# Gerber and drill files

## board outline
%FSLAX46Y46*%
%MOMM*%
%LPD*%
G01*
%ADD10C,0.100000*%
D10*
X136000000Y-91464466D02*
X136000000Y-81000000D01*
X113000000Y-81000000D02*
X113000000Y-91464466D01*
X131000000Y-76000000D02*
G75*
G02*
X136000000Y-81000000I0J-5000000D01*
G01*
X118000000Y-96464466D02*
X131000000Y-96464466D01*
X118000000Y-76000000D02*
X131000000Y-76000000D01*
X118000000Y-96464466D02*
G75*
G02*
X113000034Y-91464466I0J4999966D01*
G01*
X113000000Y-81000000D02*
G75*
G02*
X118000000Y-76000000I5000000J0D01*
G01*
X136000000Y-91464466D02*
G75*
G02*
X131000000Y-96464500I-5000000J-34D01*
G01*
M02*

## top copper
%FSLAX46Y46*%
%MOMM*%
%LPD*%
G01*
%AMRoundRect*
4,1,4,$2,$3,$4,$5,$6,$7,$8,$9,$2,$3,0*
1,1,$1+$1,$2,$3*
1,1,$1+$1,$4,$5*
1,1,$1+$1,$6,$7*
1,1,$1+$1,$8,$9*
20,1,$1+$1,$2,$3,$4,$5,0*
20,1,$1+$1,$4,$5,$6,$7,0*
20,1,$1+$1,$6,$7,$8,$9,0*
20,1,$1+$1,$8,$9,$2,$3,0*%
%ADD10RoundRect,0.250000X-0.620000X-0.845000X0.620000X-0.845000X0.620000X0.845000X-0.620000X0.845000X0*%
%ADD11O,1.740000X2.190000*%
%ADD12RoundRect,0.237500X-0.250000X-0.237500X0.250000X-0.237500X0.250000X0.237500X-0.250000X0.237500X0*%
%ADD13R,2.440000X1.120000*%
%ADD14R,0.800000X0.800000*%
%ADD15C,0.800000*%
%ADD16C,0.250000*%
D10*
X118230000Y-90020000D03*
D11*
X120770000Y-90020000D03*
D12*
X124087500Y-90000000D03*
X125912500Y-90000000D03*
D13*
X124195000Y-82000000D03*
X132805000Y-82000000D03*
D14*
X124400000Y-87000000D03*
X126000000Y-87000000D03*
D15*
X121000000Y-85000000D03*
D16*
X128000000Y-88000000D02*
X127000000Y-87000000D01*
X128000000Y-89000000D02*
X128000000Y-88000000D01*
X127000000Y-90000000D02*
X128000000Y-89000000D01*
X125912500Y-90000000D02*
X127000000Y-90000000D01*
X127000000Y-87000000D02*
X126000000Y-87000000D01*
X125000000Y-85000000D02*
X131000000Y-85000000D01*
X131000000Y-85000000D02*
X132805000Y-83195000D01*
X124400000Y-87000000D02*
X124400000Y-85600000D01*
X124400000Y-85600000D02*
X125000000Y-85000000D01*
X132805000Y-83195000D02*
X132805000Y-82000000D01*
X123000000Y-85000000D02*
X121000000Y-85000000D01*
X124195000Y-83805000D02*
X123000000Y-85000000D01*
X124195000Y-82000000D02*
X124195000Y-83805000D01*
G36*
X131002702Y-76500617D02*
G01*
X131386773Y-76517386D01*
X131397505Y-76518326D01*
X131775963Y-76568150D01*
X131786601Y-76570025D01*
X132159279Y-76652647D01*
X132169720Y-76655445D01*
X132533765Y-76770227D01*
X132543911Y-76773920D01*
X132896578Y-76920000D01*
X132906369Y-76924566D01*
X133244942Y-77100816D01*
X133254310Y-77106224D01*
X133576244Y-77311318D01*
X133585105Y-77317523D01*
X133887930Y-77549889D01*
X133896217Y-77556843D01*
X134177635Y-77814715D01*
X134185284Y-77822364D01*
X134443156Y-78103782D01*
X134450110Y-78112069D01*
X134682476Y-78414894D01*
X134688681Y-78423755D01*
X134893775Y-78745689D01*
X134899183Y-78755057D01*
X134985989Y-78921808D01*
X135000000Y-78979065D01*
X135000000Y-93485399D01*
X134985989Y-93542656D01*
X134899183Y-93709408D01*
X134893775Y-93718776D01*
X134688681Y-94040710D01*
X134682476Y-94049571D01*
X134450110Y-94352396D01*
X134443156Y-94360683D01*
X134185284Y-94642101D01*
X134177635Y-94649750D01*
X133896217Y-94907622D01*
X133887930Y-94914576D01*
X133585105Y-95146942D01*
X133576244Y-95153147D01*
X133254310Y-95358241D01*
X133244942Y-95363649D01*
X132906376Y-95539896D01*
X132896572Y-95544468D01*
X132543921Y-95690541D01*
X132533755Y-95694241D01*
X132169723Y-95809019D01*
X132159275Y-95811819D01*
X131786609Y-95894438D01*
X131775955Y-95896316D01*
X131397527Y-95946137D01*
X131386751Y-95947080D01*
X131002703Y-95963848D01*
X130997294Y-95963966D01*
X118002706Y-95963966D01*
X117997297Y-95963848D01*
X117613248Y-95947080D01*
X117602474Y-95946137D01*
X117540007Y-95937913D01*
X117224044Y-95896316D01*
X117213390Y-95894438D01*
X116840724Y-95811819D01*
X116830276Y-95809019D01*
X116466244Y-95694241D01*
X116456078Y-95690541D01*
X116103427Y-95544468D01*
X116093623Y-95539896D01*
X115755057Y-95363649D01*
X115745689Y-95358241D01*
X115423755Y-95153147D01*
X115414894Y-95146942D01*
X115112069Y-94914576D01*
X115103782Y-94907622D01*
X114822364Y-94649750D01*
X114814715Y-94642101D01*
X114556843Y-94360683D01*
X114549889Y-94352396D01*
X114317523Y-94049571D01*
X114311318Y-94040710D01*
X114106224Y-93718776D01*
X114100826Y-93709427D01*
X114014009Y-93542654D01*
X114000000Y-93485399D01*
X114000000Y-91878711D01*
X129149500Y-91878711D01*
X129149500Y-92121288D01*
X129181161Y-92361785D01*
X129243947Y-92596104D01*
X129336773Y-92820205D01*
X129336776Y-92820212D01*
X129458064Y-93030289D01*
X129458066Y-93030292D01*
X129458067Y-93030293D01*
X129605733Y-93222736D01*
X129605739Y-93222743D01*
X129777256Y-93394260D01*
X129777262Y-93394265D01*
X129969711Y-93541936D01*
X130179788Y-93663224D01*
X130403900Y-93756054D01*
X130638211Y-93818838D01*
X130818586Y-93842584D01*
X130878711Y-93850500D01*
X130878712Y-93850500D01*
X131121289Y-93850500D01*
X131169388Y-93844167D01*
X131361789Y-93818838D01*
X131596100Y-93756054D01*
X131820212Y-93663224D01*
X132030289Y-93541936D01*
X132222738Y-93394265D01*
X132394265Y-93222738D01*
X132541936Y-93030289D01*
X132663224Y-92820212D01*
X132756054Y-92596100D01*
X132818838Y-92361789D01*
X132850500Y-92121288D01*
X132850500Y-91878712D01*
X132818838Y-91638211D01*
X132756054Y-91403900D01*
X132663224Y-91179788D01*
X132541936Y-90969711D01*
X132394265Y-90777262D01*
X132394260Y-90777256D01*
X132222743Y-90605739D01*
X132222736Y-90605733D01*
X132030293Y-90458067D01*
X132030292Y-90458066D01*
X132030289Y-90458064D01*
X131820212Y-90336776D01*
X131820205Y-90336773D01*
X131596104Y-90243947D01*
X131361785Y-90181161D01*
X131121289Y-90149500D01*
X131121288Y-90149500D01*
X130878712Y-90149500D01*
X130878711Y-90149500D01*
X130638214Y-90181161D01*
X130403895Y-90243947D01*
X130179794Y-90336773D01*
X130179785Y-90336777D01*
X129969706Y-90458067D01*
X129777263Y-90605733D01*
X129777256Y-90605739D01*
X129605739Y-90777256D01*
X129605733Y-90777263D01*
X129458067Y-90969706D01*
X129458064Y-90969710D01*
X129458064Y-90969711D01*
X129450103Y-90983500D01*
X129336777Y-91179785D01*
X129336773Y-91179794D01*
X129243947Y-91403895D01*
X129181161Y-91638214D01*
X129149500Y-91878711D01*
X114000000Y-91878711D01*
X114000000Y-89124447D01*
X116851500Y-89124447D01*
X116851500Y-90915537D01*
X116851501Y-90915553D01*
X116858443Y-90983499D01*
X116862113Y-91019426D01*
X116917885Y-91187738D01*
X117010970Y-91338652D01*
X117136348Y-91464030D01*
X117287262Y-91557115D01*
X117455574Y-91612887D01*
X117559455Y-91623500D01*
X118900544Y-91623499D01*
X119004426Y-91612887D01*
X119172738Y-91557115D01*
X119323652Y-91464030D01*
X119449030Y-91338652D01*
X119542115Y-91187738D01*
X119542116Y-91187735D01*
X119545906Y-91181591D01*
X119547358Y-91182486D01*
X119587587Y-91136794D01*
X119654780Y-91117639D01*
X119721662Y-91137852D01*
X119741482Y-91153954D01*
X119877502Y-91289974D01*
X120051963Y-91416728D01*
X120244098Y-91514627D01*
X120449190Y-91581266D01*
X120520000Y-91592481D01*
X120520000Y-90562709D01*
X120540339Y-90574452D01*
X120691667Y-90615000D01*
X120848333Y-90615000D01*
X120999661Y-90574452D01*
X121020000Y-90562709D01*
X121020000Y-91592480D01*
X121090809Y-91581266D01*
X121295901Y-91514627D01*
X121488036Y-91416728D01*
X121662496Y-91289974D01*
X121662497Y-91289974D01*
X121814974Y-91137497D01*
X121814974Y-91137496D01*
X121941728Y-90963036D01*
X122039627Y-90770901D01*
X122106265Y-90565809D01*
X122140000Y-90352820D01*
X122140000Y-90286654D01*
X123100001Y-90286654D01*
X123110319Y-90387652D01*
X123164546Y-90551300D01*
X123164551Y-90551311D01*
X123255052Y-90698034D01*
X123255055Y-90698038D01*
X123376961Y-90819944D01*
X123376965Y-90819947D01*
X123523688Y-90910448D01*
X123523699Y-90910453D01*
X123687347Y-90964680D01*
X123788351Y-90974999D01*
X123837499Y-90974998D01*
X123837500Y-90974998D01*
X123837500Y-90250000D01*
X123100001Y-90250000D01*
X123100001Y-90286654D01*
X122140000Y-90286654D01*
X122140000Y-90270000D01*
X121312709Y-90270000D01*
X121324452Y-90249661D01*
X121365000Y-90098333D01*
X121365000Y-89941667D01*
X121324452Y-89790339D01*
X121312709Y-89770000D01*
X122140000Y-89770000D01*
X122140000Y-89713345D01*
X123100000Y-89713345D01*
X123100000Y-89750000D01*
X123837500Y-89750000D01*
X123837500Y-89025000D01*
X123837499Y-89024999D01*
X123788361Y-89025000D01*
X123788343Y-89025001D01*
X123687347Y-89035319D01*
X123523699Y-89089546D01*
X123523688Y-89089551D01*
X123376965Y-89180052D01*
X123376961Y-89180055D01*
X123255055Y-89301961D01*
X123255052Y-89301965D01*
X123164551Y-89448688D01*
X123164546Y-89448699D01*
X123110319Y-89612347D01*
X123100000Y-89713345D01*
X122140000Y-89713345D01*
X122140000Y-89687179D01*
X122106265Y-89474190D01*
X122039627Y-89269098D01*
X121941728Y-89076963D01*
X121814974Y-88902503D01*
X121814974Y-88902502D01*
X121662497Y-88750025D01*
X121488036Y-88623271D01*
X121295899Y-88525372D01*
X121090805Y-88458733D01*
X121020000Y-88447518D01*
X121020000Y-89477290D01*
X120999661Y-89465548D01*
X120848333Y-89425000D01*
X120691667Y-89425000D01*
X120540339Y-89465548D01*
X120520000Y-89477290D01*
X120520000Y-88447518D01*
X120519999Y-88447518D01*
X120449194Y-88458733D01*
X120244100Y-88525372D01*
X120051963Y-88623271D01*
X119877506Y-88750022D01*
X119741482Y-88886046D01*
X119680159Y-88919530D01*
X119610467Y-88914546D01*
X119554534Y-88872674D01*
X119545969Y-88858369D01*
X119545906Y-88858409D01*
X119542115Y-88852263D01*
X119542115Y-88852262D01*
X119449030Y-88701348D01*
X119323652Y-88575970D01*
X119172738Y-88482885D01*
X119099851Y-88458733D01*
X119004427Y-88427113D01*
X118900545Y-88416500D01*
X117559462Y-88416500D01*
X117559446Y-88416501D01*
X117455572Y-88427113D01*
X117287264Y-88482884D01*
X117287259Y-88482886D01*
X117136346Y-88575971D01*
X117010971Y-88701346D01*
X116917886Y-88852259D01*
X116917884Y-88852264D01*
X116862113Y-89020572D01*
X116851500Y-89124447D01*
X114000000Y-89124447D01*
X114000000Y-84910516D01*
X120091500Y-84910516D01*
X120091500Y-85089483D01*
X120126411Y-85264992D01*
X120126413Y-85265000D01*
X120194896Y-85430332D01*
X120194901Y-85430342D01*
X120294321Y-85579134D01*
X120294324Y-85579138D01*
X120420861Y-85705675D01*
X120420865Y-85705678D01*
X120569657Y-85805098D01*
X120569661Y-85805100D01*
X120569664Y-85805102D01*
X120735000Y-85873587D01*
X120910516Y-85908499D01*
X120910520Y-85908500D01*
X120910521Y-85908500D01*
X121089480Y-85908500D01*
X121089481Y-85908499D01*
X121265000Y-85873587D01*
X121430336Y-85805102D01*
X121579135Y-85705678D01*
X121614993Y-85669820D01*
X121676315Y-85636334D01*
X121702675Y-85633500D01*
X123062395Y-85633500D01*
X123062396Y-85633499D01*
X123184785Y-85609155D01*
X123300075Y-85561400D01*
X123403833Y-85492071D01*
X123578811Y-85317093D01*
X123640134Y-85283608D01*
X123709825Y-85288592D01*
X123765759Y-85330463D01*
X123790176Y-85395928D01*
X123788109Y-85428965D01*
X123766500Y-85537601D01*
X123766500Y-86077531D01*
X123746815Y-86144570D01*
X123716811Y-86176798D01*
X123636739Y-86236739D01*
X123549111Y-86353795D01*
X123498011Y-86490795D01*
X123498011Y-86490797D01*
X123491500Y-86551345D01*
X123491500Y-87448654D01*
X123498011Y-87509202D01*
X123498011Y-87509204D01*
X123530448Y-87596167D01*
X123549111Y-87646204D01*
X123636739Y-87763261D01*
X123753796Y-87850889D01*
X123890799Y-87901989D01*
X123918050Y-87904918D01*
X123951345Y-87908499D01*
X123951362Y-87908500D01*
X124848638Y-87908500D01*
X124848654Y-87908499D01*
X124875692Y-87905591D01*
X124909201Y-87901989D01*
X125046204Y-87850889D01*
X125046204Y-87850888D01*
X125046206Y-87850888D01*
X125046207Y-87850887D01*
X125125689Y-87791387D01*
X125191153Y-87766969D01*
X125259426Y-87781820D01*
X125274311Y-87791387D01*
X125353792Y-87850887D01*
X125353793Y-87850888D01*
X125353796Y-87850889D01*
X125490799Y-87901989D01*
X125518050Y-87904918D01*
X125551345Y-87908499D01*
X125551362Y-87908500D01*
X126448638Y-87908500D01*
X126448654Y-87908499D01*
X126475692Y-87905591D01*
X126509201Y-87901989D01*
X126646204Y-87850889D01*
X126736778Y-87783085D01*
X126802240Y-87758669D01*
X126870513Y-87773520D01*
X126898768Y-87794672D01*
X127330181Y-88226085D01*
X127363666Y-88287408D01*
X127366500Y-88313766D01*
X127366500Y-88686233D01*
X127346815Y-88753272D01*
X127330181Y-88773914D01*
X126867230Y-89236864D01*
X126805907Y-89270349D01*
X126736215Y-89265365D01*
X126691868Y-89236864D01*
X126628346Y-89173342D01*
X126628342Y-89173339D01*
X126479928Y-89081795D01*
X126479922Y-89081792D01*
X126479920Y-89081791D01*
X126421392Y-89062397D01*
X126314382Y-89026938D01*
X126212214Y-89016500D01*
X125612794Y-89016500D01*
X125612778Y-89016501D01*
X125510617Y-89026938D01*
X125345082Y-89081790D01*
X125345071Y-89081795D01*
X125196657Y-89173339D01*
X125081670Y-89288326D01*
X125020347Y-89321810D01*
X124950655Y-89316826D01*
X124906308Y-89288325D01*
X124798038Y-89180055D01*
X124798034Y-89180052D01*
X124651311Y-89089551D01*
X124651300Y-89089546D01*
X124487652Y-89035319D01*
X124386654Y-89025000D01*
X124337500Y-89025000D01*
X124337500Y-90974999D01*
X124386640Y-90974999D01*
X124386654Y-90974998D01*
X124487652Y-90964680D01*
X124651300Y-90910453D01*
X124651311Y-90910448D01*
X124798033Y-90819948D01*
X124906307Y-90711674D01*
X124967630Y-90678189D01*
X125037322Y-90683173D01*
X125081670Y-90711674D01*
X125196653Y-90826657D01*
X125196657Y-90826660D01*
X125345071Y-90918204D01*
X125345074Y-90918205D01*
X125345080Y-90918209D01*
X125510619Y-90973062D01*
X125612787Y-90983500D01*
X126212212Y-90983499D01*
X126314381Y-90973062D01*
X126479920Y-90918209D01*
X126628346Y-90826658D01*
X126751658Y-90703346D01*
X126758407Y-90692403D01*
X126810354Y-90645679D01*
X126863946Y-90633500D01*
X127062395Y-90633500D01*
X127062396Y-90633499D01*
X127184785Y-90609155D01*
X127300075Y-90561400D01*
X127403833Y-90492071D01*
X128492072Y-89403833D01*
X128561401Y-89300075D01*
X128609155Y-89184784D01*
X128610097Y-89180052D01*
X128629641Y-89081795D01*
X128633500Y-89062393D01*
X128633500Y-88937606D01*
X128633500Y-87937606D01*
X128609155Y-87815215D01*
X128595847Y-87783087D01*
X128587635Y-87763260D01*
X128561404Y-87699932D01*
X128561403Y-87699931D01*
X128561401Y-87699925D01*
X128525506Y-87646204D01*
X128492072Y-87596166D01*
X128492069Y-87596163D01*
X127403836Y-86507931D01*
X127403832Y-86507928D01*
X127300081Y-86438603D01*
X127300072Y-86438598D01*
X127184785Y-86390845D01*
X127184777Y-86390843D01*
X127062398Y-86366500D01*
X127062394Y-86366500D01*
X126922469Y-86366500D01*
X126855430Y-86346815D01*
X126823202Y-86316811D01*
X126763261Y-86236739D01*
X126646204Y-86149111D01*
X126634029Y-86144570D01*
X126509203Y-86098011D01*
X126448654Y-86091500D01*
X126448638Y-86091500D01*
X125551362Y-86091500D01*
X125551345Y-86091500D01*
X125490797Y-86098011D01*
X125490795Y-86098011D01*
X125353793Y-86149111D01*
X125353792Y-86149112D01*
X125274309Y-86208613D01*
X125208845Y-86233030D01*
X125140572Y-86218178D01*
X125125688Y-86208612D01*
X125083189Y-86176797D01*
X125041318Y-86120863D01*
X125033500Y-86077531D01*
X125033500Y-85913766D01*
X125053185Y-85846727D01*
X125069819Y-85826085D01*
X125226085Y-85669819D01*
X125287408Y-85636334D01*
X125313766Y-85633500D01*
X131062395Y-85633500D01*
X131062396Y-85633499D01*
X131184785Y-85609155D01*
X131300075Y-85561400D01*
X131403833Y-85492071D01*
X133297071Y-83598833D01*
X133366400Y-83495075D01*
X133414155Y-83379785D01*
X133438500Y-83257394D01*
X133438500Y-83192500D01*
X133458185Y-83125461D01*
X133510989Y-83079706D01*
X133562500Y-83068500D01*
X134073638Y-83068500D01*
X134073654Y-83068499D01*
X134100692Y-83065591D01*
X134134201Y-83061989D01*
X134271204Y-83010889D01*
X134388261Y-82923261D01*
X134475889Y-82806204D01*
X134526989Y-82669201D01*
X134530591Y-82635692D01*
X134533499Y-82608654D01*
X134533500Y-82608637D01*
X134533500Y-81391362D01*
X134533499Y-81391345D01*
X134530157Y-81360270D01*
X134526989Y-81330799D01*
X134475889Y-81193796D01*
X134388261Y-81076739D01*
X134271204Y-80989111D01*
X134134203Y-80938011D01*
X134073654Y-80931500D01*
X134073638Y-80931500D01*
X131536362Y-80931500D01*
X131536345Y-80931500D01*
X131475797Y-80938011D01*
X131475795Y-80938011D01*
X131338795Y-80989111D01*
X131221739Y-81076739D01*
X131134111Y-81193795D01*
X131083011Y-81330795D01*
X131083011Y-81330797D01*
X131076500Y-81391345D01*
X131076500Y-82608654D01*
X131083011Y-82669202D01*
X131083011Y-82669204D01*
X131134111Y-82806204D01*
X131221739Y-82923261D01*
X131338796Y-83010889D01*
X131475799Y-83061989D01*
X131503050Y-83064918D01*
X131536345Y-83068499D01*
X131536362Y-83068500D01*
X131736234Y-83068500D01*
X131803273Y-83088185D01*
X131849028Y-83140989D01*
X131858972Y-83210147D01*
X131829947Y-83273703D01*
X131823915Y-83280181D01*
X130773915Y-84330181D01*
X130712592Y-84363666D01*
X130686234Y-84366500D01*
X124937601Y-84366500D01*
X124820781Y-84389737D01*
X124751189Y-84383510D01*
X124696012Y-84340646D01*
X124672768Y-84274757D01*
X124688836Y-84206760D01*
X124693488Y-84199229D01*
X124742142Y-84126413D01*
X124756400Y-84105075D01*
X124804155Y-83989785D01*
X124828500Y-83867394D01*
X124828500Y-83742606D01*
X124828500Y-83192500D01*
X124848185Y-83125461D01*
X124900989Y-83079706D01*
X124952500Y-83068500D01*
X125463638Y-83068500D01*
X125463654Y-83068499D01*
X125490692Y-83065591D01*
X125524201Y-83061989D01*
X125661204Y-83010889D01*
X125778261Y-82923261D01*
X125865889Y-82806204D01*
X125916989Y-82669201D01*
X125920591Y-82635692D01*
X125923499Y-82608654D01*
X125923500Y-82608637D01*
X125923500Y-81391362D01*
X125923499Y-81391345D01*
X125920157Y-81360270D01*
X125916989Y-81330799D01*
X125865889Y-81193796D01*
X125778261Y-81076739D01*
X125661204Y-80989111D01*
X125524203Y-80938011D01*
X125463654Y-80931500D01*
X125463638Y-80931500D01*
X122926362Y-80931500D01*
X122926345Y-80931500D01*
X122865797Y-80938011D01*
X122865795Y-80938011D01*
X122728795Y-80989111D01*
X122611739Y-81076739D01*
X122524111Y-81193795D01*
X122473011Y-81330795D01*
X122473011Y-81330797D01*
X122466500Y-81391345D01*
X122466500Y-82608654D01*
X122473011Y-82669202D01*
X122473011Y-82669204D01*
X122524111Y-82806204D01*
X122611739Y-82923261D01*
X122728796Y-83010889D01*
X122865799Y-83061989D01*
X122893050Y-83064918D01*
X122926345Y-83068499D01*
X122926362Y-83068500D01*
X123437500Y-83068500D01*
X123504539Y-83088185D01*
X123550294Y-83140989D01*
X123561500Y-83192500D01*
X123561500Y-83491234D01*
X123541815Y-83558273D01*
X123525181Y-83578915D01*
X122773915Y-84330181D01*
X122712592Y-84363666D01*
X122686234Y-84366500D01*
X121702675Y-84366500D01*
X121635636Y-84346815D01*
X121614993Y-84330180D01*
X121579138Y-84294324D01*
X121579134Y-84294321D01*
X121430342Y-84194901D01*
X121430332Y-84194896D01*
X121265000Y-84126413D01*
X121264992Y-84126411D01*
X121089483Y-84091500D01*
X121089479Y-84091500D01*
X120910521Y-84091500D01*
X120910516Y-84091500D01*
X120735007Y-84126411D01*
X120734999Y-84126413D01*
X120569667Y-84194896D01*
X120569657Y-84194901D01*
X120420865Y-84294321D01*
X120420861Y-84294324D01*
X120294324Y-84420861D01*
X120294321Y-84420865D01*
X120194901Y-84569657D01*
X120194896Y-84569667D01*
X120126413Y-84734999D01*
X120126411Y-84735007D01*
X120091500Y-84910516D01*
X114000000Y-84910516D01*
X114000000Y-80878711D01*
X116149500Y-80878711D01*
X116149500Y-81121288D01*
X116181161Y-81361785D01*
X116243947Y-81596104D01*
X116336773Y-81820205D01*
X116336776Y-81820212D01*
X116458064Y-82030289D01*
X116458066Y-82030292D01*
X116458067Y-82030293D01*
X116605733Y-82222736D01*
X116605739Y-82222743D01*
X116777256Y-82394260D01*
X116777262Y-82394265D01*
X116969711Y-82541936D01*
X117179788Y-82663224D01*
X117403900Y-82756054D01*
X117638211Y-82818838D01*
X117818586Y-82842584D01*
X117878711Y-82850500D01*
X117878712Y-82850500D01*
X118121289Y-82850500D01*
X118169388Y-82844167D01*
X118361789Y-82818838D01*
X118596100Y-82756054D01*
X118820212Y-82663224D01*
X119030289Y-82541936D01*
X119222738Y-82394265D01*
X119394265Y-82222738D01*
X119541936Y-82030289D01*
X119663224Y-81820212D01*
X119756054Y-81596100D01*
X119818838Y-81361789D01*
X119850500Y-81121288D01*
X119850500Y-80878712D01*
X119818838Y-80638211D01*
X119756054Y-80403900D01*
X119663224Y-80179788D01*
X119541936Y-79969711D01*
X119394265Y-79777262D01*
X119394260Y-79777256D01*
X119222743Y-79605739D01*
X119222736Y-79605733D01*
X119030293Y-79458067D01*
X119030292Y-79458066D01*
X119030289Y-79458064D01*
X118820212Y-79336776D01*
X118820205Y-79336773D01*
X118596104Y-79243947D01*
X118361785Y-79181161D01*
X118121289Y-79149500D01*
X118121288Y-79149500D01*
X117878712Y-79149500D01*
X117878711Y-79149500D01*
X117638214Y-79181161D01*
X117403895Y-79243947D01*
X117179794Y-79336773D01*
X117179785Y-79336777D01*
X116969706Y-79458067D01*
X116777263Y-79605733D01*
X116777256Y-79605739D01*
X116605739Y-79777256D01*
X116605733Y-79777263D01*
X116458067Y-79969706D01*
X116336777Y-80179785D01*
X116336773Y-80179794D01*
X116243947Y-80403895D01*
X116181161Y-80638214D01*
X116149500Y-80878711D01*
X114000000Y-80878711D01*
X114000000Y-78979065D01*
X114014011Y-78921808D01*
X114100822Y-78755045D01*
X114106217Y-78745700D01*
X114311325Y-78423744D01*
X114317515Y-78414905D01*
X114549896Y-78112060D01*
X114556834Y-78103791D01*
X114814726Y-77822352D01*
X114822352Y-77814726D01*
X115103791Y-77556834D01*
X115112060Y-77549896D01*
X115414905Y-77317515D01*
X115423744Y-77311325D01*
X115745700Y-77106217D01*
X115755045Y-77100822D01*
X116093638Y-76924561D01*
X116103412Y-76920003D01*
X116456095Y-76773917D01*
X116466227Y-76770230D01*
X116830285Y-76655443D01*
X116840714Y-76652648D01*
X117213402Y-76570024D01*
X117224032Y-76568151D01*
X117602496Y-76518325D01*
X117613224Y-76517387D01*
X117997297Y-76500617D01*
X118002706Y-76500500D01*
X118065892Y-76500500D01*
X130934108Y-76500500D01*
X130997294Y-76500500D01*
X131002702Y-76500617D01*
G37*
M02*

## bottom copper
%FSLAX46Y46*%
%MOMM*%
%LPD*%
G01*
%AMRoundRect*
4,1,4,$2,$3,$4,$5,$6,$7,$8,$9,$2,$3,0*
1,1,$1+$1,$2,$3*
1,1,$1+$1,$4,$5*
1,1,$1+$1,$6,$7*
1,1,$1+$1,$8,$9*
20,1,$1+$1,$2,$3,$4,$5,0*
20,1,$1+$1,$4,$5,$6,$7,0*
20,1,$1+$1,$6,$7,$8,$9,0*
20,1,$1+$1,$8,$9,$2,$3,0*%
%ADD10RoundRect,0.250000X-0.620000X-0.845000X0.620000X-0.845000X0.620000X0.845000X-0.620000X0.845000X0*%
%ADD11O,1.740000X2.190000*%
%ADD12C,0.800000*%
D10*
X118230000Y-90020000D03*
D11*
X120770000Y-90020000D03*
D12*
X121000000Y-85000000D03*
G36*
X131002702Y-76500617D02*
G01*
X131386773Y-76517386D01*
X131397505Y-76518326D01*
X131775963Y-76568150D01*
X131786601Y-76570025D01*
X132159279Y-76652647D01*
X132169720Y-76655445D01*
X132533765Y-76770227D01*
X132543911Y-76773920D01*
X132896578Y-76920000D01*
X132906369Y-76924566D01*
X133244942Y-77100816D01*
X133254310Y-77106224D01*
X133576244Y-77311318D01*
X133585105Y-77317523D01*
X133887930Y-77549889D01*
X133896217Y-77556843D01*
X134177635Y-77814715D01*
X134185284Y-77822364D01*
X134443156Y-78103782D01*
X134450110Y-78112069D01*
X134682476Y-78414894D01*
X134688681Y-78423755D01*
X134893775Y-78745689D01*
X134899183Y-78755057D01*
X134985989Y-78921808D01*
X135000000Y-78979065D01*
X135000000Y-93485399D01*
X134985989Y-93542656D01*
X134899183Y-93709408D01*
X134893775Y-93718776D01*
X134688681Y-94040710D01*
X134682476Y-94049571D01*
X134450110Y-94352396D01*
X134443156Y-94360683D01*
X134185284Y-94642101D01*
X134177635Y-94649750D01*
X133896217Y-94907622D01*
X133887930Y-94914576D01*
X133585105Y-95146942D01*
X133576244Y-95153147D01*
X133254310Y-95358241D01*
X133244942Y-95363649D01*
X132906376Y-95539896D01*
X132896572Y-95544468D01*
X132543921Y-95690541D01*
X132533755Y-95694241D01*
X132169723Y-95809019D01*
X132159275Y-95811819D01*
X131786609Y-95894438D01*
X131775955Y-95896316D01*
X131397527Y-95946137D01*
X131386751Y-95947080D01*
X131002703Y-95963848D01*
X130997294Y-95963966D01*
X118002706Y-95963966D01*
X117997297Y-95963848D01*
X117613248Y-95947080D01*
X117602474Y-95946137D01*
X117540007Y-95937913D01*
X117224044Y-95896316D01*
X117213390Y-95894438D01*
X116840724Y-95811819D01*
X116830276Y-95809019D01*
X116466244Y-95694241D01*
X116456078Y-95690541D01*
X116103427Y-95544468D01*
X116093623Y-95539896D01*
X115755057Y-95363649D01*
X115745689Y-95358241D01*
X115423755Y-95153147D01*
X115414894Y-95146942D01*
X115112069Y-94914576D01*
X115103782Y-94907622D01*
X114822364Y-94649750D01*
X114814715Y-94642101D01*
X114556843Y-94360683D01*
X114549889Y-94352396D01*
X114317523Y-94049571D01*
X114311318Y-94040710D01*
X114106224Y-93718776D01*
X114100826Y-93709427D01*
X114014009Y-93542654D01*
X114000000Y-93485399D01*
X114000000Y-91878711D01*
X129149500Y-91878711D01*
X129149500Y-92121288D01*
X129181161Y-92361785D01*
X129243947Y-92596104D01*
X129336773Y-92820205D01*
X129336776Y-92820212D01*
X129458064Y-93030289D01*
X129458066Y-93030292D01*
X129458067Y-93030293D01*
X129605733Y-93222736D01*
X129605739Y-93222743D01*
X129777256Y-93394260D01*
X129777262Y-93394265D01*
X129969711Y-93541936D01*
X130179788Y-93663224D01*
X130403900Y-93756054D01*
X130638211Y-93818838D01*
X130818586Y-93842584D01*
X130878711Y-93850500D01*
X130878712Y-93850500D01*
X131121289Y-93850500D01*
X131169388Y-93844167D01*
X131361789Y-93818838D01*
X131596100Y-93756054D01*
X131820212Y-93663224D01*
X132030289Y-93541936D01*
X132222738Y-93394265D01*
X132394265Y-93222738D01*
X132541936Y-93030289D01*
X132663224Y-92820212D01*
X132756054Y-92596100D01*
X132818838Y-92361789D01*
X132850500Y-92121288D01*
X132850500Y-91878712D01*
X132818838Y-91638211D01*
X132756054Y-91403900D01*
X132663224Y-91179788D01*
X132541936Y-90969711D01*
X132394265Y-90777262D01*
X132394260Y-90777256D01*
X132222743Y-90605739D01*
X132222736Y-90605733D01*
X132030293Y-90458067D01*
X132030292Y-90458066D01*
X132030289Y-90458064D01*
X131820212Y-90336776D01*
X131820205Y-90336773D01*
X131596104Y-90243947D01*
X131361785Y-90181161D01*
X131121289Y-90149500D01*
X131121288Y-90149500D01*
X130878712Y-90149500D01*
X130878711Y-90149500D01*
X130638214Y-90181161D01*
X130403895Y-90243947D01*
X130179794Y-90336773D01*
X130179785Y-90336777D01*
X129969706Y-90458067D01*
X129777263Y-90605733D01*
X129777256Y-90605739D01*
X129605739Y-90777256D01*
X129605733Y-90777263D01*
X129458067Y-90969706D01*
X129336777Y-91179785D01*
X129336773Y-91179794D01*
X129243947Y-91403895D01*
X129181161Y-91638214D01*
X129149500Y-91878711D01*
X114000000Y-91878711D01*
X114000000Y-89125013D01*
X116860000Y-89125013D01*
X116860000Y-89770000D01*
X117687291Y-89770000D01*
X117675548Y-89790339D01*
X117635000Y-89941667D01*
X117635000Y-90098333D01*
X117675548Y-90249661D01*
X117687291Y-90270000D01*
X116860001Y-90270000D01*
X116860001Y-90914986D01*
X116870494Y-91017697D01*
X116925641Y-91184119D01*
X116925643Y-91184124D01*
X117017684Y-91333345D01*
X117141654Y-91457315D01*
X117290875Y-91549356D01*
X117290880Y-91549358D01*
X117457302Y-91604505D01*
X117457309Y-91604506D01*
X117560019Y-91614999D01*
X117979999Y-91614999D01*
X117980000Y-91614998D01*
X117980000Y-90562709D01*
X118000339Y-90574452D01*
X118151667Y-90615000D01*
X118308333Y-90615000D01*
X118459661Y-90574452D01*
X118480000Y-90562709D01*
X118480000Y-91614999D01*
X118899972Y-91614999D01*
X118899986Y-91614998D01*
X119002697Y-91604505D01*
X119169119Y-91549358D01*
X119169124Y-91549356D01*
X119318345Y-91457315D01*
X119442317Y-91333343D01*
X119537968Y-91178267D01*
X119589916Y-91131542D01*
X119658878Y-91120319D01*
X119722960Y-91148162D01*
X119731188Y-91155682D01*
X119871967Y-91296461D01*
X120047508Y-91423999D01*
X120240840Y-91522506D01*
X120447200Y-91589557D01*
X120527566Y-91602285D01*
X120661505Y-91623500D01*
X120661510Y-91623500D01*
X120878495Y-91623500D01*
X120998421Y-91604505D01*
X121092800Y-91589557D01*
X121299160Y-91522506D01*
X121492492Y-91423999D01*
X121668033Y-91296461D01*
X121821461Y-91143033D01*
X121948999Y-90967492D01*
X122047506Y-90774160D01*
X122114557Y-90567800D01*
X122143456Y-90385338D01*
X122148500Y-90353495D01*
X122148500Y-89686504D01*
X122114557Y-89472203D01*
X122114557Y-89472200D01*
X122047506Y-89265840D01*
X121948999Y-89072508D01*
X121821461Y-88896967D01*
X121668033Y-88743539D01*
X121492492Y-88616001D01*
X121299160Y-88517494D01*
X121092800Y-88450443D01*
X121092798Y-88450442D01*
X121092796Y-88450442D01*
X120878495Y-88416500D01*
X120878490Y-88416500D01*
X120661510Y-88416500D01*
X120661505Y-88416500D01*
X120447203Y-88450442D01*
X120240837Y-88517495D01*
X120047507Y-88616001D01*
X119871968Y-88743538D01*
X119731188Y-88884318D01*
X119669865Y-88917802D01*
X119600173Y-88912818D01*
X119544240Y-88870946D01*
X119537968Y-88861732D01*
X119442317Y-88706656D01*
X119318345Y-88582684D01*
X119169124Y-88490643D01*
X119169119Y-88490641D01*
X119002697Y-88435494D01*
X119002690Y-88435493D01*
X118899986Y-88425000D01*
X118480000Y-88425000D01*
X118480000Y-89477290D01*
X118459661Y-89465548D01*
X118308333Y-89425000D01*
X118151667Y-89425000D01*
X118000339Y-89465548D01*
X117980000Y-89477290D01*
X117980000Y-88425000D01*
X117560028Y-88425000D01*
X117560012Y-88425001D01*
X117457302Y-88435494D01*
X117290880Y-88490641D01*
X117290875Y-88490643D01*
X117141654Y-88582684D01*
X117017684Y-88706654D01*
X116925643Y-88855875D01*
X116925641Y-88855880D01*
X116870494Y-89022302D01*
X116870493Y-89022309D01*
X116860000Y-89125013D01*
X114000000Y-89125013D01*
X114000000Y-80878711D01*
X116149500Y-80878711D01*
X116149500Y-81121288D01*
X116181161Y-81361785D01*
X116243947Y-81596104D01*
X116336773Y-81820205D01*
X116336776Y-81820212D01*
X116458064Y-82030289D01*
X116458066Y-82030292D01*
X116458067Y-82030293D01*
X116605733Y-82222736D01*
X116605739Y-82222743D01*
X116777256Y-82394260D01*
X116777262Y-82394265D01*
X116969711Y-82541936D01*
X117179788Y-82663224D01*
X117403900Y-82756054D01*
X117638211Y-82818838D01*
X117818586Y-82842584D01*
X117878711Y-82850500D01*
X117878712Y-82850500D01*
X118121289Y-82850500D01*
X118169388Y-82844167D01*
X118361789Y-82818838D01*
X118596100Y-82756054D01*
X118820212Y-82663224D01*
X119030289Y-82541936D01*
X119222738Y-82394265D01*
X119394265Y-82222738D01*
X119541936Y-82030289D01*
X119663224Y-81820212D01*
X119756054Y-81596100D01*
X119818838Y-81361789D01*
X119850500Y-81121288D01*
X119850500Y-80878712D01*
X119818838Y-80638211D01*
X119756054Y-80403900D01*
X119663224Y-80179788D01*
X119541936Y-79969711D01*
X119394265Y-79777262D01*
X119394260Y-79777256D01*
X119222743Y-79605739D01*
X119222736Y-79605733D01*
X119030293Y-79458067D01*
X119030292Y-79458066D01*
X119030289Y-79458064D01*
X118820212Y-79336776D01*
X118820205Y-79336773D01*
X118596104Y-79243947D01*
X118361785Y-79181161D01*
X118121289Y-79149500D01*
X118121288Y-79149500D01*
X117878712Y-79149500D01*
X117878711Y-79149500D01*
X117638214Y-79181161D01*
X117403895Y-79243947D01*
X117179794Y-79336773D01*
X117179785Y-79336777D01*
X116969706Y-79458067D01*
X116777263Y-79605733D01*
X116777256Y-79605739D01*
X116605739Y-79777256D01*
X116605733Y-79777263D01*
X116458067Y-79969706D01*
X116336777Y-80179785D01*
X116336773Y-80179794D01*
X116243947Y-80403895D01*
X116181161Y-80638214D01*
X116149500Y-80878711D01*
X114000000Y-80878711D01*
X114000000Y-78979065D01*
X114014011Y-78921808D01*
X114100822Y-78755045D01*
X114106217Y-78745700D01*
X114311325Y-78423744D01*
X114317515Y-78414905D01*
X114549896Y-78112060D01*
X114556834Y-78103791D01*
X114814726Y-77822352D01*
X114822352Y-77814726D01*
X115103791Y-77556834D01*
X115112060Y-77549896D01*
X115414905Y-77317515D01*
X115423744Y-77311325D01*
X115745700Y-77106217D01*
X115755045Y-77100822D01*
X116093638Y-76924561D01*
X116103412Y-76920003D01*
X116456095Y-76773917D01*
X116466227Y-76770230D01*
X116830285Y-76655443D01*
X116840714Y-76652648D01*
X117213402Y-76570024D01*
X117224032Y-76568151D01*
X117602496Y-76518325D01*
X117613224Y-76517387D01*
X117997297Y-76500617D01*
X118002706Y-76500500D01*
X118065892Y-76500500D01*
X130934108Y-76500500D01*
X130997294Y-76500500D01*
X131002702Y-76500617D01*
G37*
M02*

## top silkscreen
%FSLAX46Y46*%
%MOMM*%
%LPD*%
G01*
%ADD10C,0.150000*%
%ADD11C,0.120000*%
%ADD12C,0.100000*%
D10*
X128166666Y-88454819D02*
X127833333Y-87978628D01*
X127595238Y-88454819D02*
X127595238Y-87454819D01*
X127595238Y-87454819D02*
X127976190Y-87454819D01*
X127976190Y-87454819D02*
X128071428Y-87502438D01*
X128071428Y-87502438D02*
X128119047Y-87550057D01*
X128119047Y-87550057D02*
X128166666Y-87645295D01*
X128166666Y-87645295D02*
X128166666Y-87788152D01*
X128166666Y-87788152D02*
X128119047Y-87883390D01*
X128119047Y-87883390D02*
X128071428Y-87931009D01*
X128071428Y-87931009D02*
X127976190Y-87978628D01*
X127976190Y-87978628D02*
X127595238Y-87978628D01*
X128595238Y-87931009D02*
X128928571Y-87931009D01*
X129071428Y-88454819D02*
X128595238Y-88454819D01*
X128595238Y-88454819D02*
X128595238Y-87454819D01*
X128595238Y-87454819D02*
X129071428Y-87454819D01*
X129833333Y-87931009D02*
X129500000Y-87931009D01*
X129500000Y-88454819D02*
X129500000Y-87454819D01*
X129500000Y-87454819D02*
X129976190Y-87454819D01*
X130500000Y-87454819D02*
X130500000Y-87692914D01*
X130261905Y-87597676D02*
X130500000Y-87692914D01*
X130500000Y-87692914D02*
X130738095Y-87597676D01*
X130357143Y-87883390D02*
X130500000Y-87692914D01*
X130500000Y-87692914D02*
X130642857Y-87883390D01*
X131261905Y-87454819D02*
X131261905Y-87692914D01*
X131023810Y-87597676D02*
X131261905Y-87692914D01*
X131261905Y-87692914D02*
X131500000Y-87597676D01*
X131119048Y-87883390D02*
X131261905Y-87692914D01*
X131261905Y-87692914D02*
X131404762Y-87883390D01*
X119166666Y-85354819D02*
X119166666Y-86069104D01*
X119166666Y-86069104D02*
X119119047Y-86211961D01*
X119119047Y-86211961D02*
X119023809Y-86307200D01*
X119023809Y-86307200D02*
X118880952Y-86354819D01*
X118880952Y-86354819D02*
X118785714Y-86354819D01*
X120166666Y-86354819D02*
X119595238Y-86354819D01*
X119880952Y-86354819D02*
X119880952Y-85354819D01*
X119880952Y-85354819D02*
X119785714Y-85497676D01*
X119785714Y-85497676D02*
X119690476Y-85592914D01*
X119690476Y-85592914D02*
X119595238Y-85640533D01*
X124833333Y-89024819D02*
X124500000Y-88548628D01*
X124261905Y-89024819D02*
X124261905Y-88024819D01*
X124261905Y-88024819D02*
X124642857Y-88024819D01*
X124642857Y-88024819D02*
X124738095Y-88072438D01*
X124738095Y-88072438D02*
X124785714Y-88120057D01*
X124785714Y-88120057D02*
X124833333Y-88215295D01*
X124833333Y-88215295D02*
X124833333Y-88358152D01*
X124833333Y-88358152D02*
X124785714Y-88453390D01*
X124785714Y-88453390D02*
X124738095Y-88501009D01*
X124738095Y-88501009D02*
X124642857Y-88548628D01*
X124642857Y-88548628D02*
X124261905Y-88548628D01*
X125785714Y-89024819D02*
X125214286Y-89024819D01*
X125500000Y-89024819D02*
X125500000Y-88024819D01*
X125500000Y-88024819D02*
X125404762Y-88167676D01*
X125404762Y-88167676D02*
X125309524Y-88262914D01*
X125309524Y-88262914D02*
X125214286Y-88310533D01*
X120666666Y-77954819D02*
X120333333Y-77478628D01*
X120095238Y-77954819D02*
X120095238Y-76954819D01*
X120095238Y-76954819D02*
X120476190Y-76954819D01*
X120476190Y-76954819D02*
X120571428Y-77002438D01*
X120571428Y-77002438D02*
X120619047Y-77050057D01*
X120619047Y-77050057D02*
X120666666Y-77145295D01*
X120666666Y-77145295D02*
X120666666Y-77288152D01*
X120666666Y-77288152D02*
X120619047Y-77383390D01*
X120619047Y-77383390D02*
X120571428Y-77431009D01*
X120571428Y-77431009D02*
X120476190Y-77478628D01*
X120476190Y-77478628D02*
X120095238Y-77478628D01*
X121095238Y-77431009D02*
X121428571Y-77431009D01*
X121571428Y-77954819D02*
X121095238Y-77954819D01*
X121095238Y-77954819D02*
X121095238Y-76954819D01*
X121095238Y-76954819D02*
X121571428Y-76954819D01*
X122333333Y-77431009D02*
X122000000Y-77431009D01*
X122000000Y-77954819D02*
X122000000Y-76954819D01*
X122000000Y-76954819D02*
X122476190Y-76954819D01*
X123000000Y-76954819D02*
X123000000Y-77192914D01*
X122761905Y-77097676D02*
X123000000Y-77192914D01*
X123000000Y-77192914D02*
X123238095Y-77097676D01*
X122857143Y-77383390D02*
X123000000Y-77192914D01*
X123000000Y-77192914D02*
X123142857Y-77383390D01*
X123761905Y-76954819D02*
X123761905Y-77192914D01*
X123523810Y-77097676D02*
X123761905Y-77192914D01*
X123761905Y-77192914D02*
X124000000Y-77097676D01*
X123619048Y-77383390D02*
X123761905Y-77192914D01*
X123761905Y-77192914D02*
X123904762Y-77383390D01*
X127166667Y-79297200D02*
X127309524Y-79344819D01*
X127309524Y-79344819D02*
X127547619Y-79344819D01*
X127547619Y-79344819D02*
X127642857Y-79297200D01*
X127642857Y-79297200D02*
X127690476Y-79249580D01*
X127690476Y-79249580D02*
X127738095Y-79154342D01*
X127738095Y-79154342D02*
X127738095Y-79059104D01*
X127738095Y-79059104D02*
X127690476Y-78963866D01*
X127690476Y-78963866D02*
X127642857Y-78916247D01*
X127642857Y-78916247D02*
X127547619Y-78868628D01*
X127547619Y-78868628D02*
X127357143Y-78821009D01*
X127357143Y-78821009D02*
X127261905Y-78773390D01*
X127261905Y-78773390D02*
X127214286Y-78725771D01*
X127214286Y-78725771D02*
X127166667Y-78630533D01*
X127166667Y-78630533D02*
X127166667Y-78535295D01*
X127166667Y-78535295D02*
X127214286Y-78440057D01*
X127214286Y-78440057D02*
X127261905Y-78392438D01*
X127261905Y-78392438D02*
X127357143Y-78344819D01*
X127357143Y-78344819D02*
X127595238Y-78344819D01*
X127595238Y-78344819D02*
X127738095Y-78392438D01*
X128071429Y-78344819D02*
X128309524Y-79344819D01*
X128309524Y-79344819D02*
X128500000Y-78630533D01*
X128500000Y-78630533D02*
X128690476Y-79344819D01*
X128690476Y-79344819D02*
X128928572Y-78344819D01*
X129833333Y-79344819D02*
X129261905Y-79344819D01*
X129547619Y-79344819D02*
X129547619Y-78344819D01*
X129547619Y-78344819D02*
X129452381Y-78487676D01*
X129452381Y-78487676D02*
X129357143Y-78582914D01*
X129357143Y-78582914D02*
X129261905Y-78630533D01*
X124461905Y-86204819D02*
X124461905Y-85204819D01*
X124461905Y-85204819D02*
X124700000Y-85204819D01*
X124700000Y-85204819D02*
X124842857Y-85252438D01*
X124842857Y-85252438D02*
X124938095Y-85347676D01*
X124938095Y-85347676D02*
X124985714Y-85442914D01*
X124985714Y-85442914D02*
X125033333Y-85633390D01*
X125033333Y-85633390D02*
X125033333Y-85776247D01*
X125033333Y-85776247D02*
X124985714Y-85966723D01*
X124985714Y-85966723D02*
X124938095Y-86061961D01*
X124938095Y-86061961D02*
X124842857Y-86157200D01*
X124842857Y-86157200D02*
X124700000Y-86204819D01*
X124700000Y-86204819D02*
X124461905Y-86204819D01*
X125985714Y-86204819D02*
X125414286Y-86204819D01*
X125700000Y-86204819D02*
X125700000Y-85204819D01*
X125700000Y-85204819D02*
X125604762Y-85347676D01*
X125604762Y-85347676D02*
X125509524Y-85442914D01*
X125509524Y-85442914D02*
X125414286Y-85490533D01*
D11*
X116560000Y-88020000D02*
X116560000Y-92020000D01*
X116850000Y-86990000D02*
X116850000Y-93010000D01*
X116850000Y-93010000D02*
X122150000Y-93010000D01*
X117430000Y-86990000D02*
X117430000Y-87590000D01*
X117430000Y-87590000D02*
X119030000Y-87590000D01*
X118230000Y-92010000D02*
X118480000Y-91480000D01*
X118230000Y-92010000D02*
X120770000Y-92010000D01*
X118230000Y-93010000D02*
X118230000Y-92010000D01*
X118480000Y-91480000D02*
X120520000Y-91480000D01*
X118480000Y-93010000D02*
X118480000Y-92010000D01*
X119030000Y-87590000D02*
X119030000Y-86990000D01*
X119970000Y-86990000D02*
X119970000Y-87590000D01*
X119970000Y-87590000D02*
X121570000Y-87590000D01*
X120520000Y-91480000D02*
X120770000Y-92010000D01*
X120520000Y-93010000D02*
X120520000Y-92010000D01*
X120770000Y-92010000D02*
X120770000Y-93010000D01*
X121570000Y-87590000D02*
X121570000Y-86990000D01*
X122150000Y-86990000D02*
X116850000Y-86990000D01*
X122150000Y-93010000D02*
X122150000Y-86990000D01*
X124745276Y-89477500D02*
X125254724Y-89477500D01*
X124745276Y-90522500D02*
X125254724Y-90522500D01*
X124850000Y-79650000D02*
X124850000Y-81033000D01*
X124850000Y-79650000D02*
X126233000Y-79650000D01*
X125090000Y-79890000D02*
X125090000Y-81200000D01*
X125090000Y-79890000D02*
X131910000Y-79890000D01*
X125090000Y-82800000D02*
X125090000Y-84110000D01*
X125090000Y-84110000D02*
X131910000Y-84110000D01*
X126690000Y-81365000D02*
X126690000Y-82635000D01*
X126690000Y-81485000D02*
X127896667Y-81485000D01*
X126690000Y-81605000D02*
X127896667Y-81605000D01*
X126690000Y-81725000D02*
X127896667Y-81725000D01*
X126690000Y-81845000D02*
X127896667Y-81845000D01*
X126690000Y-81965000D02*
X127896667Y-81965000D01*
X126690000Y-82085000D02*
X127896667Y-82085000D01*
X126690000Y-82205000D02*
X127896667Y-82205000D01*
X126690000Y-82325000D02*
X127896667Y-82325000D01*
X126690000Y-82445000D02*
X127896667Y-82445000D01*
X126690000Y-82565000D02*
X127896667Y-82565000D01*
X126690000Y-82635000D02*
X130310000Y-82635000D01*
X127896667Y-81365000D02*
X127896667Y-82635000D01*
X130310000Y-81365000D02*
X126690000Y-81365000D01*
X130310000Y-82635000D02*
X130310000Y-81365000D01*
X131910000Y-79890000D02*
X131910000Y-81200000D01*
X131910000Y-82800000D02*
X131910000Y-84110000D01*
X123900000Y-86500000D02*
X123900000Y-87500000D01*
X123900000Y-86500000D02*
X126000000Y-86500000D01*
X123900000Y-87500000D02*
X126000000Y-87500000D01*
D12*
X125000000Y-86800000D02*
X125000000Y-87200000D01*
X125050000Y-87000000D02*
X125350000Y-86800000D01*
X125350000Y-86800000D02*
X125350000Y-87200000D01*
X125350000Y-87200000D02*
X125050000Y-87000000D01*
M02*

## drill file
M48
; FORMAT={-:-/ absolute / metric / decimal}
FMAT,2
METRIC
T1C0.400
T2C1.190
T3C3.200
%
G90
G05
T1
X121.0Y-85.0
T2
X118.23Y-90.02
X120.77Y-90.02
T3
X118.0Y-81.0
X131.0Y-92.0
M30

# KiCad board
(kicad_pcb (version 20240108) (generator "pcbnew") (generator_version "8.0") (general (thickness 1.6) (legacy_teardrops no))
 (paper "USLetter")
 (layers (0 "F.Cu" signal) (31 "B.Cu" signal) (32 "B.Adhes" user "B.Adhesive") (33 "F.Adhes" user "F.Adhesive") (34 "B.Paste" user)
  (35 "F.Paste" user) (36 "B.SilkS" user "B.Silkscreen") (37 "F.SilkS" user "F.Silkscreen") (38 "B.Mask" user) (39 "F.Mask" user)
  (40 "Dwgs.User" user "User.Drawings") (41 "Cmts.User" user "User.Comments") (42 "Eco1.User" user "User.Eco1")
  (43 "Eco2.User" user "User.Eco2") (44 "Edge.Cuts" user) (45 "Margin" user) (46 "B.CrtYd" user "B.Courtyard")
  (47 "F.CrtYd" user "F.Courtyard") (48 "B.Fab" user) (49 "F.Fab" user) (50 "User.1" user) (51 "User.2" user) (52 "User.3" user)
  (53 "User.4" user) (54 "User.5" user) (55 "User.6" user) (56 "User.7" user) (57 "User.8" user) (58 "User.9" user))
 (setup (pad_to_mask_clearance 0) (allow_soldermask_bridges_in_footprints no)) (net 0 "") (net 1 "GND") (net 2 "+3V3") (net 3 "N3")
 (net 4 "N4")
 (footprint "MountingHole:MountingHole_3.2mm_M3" (layer "F.Cu") (at 131 92)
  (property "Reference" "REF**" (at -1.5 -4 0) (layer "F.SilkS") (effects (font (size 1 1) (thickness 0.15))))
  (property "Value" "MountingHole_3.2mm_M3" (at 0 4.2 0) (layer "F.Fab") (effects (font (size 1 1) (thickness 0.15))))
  (pad "" np_thru_hole circle (at 0 0) (size 3.2 3.2) (drill 3.2) (layers "*.Cu" "*.Mask")))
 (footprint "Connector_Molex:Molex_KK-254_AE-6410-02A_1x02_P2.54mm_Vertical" (layer "F.Cu") (at 118.23 90.02)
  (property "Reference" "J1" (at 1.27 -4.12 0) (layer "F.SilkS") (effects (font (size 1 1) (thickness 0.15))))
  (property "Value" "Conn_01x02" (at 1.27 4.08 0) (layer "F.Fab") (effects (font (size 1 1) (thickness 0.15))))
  (fp_line (start -1.67 -2) (end -1.67 2) (stroke (width 0.12) (type solid)) (layer "F.SilkS"))
  (fp_line (start -1.38 -3.03) (end -1.38 2.99) (stroke (width 0.12) (type solid)) (layer "F.SilkS"))
  (fp_line (start -1.38 2.99) (end 3.92 2.99) (stroke (width 0.12) (type solid)) (layer "F.SilkS"))
  (fp_line (start -0.8 -3.03) (end -0.8 -2.43) (stroke (width 0.12) (type solid)) (layer "F.SilkS"))
  (fp_line (start -0.8 -2.43) (end 0.8 -2.43) (stroke (width 0.12) (type solid)) (layer "F.SilkS"))
  (fp_line (start 0 1.99) (end 0.25 1.46) (stroke (width 0.12) (type solid)) (layer "F.SilkS"))
  (fp_line (start 0 1.99) (end 2.54 1.99) (stroke (width 0.12) (type solid)) (layer "F.SilkS"))
  (fp_line (start 0 2.99) (end 0 1.99) (stroke (width 0.12) (type solid)) (layer "F.SilkS"))
  (fp_line (start 0.25 1.46) (end 2.29 1.46) (stroke (width 0.12) (type solid)) (layer "F.SilkS"))
  (fp_line (start 0.25 2.99) (end 0.25 1.99) (stroke (width 0.12) (type solid)) (layer "F.SilkS"))
  (fp_line (start 0.8 -2.43) (end 0.8 -3.03) (stroke (width 0.12) (type solid)) (layer "F.SilkS"))
  (fp_line (start 1.74 -3.03) (end 1.74 -2.43) (stroke (width 0.12) (type solid)) (layer "F.SilkS"))
  (fp_line (start 1.74 -2.43) (end 3.34 -2.43) (stroke (width 0.12) (type solid)) (layer "F.SilkS"))
  (fp_line (start 2.29 1.46) (end 2.54 1.99) (stroke (width 0.12) (type solid)) (layer "F.SilkS"))
  (fp_line (start 2.29 2.99) (end 2.29 1.99) (stroke (width 0.12) (type solid)) (layer "F.SilkS"))
  (fp_line (start 2.54 1.99) (end 2.54 2.99) (stroke (width 0.12) (type solid)) (layer "F.SilkS"))
  (fp_line (start 3.34 -2.43) (end 3.34 -3.03) (stroke (width 0.12) (type solid)) (layer "F.SilkS"))
  (fp_line (start 3.92 -3.03) (end -1.38 -3.03) (stroke (width 0.12) (type solid)) (layer "F.SilkS"))
  (fp_line (start 3.92 2.99) (end 3.92 -3.03) (stroke (width 0.12) (type solid)) (layer "F.SilkS"))
  (pad "1" thru_hole roundrect (at 0 0) (size 1.74 2.19) (drill 1.19) (layers "*.Cu" "*.Mask") (remove_unused_layers no)
   (roundrect_rratio 0.143678) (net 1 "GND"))
  (pad "2" thru_hole oval (at 2.54 0) (size 1.74 2.19) (drill 1.19) (layers "*.Cu" "*.Mask") (remove_unused_layers no) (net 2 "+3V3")))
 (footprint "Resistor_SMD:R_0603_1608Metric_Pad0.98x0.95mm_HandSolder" (layer "F.Cu") (at 125 90)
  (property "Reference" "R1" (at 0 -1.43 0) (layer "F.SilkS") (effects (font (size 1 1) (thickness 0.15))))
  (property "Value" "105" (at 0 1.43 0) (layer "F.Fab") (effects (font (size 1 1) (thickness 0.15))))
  (fp_line (start -0.254724 -0.5225) (end 0.254724 -0.5225) (stroke (width 0.12) (type solid)) (layer "F.SilkS"))
  (fp_line (start -0.254724 0.5225) (end 0.254724 0.5225) (stroke (width 0.12) (type solid)) (layer "F.SilkS"))
  (pad "1" smd roundrect (at -0.9125 0) (size 0.975 0.95) (layers "F.Cu" "F.Paste" "F.Mask") (roundrect_rratio 0.25) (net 2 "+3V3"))
  (pad "2" smd roundrect (at 0.9125 0) (size 0.975 0.95) (layers "F.Cu" "F.Paste" "F.Mask") (roundrect_rratio 0.25) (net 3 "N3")))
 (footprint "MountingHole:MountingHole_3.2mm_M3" (layer "F.Cu") (at 118 81)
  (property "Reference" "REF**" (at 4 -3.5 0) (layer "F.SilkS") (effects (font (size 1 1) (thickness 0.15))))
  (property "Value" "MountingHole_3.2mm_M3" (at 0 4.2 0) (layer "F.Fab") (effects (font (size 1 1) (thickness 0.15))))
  (pad "" np_thru_hole circle (at 0 0) (size 3.2 3.2) (drill 3.2) (layers "*.Cu" "*.Mask")))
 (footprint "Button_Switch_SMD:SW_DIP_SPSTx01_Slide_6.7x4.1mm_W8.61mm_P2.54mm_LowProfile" (layer "F.Cu") (at 128.5 82)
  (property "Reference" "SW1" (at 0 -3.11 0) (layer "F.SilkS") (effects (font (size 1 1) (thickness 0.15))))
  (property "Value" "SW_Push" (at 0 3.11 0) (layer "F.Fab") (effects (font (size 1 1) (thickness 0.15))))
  (fp_line (start -3.65 -2.35) (end -3.65 -0.967) (stroke (width 0.12) (type solid)) (layer "F.SilkS"))
  (fp_line (start -3.65 -2.35) (end -2.267 -2.35) (stroke (width 0.12) (type solid)) (layer "F.SilkS"))
  (fp_line (start -3.41 -2.11) (end -3.41 -0.8) (stroke (width 0.12) (type solid)) (layer "F.SilkS"))
  (fp_line (start -3.41 -2.11) (end 3.41 -2.11) (stroke (width 0.12) (type solid)) (layer "F.SilkS"))
  (fp_line (start -3.41 0.8) (end -3.41 2.11) (stroke (width 0.12) (type solid)) (layer "F.SilkS"))
  (fp_line (start -3.41 2.11) (end 3.41 2.11) (stroke (width 0.12) (type solid)) (layer "F.SilkS"))
  (fp_line (start -1.81 -0.635) (end -1.81 0.635) (stroke (width 0.12) (type solid)) (layer "F.SilkS"))
  (fp_line (start -1.81 -0.515) (end -0.603333 -0.515) (stroke (width 0.12) (type solid)) (layer "F.SilkS"))
  (fp_line (start -1.81 -0.395) (end -0.603333 -0.395) (stroke (width 0.12) (type solid)) (layer "F.SilkS"))
  (fp_line (start -1.81 -0.275) (end -0.603333 -0.275) (stroke (width 0.12) (type solid)) (layer "F.SilkS"))
  (fp_line (start -1.81 -0.155) (end -0.603333 -0.155) (stroke (width 0.12) (type solid)) (layer "F.SilkS"))
  (fp_line (start -1.81 -0.035) (end -0.603333 -0.035) (stroke (width 0.12) (type solid)) (layer "F.SilkS"))
  (fp_line (start -1.81 0.085) (end -0.603333 0.085) (stroke (width 0.12) (type solid)) (layer "F.SilkS"))
  (fp_line (start -1.81 0.205) (end -0.603333 0.205) (stroke (width 0.12) (type solid)) (layer "F.SilkS"))
  (fp_line (start -1.81 0.325) (end -0.603333 0.325) (stroke (width 0.12) (type solid)) (layer "F.SilkS"))
  (fp_line (start -1.81 0.445) (end -0.603333 0.445) (stroke (width 0.12) (type solid)) (layer "F.SilkS"))
  (fp_line (start -1.81 0.565) (end -0.603333 0.565) (stroke (width 0.12) (type solid)) (layer "F.SilkS"))
  (fp_line (start -1.81 0.635) (end 1.81 0.635) (stroke (width 0.12) (type solid)) (layer "F.SilkS"))
  (fp_line (start -0.603333 -0.635) (end -0.603333 0.635) (stroke (width 0.12) (type solid)) (layer "F.SilkS"))
  (fp_line (start 1.81 -0.635) (end -1.81 -0.635) (stroke (width 0.12) (type solid)) (layer "F.SilkS"))
  (fp_line (start 1.81 0.635) (end 1.81 -0.635) (stroke (width 0.12) (type solid)) (layer "F.SilkS"))
  (fp_line (start 3.41 -2.11) (end 3.41 -0.8) (stroke (width 0.12) (type solid)) (layer "F.SilkS"))
  (fp_line (start 3.41 0.8) (end 3.41 2.11) (stroke (width 0.12) (type solid)) (layer "F.SilkS"))
  (pad "1" smd rect (at -4.305 0) (size 2.44 1.12) (layers "F.Cu" "F.Paste" "F.Mask") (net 1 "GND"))
  (pad "2" smd rect (at 4.305 0) (size 2.44 1.12) (layers "F.Cu" "F.Paste" "F.Mask") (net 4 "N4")))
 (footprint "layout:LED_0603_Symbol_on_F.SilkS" (layer "F.Cu") (at 125.2 87)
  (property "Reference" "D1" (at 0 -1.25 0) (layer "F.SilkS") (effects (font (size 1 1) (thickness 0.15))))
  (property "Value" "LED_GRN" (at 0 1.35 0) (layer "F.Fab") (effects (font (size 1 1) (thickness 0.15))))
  (fp_line (start -1.3 -0.5) (end -1.3 0.5) (stroke (width 0.12) (type solid)) (layer "F.SilkS"))
  (fp_line (start -1.3 -0.5) (end 0.8 -0.5) (stroke (width 0.12) (type solid)) (layer "F.SilkS"))
  (fp_line (start -1.3 0.5) (end 0.8 0.5) (stroke (width 0.12) (type solid)) (layer "F.SilkS"))
  (fp_line (start -0.2 -0.2) (end -0.2 0.2) (stroke (width 0.1) (type solid)) (layer "F.SilkS"))
  (fp_line (start -0.15 0) (end 0.15 -0.2) (stroke (width 0.1) (type solid)) (layer "F.SilkS"))
  (fp_line (start 0.15 -0.2) (end 0.15 0.2) (stroke (width 0.1) (type solid)) (layer "F.SilkS"))
  (fp_line (start 0.15 0.2) (end -0.15 0) (stroke (width 0.1) (type solid)) (layer "F.SilkS"))
  (pad "1" smd rect (at -0.8 0 180) (size 0.8 0.8) (layers "F.Cu" "F.Paste" "F.Mask") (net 4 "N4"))
  (pad "2" smd rect (at 0.8 0 180) (size 0.8 0.8) (layers "F.Cu" "F.Paste" "F.Mask") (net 3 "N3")))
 (gr_line (start 136 91.464466) (end 136 81) (stroke (width 0.1) (type default)) (layer "Edge.Cuts"))
 (gr_line (start 113 81) (end 113 91.464466) (stroke (width 0.1) (type default)) (layer "Edge.Cuts"))
 (gr_arc (start 131 76) (mid 134.535534 77.464466) (end 136 81) (stroke (width 0.1) (type default)) (layer "Edge.Cuts"))
 (gr_line (start 118 96.464466) (end 131 96.464466) (stroke (width 0.1) (type default)) (layer "Edge.Cuts"))
 (gr_line (start 118 76) (end 131 76) (stroke (width 0.1) (type default)) (layer "Edge.Cuts"))
 (gr_arc (start 118 96.464466) (mid 114.464466 95) (end 113 91.464466) (stroke (width 0.1) (type default)) (layer "Edge.Cuts"))
 (gr_arc (start 113 81) (mid 114.464466 77.464466) (end 118 76) (stroke (width 0.1) (type default)) (layer "Edge.Cuts"))
 (gr_arc (start 136 91.464466) (mid 134.535534 95) (end 131 96.464466) (stroke (width 0.1) (type default)) (layer "Edge.Cuts"))
 (segment (start 128 88) (end 127 87) (width 0.25) (layer "F.Cu") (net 3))
 (segment (start 128 89) (end 128 88) (width 0.25) (layer "F.Cu") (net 3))
 (segment (start 127 90) (end 128 89) (width 0.25) (layer "F.Cu") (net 3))
 (segment (start 125.9125 90) (end 127 90) (width 0.25) (layer "F.Cu") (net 3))
 (segment (start 127 87) (end 126 87) (width 0.25) (layer "F.Cu") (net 3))
 (segment (start 125 85) (end 131 85) (width 0.25) (layer "F.Cu") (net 4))
 (segment (start 131 85) (end 132.805 83.195) (width 0.25) (layer "F.Cu") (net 4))
 (segment (start 124.4 87) (end 124.4 85.6) (width 0.25) (layer "F.Cu") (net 4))
 (segment (start 124.4 85.6) (end 125 85) (width 0.25) (layer "F.Cu") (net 4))
 (segment (start 132.805 83.195) (end 132.805 82) (width 0.25) (layer "F.Cu") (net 4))
 (segment (start 123 85) (end 121 85) (width 0.25) (layer "F.Cu") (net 1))
 (segment (start 124.195 83.805) (end 123 85) (width 0.25) (layer "F.Cu") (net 1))
 (segment (start 124.195 82) (end 124.195 83.805) (width 0.25) (layer "F.Cu") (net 1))
 (via (at 121 85) (size 0.8) (drill 0.4) (layers "F.Cu" "B.Cu") (free yes) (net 1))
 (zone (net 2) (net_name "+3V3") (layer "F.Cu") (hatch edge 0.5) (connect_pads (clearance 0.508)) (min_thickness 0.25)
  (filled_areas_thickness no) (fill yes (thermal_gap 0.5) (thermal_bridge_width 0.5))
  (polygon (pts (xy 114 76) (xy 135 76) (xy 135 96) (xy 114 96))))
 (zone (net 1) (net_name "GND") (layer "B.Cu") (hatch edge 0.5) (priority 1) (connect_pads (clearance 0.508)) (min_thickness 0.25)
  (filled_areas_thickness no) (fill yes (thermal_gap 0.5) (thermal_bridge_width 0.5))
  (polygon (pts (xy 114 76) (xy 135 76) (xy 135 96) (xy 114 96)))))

